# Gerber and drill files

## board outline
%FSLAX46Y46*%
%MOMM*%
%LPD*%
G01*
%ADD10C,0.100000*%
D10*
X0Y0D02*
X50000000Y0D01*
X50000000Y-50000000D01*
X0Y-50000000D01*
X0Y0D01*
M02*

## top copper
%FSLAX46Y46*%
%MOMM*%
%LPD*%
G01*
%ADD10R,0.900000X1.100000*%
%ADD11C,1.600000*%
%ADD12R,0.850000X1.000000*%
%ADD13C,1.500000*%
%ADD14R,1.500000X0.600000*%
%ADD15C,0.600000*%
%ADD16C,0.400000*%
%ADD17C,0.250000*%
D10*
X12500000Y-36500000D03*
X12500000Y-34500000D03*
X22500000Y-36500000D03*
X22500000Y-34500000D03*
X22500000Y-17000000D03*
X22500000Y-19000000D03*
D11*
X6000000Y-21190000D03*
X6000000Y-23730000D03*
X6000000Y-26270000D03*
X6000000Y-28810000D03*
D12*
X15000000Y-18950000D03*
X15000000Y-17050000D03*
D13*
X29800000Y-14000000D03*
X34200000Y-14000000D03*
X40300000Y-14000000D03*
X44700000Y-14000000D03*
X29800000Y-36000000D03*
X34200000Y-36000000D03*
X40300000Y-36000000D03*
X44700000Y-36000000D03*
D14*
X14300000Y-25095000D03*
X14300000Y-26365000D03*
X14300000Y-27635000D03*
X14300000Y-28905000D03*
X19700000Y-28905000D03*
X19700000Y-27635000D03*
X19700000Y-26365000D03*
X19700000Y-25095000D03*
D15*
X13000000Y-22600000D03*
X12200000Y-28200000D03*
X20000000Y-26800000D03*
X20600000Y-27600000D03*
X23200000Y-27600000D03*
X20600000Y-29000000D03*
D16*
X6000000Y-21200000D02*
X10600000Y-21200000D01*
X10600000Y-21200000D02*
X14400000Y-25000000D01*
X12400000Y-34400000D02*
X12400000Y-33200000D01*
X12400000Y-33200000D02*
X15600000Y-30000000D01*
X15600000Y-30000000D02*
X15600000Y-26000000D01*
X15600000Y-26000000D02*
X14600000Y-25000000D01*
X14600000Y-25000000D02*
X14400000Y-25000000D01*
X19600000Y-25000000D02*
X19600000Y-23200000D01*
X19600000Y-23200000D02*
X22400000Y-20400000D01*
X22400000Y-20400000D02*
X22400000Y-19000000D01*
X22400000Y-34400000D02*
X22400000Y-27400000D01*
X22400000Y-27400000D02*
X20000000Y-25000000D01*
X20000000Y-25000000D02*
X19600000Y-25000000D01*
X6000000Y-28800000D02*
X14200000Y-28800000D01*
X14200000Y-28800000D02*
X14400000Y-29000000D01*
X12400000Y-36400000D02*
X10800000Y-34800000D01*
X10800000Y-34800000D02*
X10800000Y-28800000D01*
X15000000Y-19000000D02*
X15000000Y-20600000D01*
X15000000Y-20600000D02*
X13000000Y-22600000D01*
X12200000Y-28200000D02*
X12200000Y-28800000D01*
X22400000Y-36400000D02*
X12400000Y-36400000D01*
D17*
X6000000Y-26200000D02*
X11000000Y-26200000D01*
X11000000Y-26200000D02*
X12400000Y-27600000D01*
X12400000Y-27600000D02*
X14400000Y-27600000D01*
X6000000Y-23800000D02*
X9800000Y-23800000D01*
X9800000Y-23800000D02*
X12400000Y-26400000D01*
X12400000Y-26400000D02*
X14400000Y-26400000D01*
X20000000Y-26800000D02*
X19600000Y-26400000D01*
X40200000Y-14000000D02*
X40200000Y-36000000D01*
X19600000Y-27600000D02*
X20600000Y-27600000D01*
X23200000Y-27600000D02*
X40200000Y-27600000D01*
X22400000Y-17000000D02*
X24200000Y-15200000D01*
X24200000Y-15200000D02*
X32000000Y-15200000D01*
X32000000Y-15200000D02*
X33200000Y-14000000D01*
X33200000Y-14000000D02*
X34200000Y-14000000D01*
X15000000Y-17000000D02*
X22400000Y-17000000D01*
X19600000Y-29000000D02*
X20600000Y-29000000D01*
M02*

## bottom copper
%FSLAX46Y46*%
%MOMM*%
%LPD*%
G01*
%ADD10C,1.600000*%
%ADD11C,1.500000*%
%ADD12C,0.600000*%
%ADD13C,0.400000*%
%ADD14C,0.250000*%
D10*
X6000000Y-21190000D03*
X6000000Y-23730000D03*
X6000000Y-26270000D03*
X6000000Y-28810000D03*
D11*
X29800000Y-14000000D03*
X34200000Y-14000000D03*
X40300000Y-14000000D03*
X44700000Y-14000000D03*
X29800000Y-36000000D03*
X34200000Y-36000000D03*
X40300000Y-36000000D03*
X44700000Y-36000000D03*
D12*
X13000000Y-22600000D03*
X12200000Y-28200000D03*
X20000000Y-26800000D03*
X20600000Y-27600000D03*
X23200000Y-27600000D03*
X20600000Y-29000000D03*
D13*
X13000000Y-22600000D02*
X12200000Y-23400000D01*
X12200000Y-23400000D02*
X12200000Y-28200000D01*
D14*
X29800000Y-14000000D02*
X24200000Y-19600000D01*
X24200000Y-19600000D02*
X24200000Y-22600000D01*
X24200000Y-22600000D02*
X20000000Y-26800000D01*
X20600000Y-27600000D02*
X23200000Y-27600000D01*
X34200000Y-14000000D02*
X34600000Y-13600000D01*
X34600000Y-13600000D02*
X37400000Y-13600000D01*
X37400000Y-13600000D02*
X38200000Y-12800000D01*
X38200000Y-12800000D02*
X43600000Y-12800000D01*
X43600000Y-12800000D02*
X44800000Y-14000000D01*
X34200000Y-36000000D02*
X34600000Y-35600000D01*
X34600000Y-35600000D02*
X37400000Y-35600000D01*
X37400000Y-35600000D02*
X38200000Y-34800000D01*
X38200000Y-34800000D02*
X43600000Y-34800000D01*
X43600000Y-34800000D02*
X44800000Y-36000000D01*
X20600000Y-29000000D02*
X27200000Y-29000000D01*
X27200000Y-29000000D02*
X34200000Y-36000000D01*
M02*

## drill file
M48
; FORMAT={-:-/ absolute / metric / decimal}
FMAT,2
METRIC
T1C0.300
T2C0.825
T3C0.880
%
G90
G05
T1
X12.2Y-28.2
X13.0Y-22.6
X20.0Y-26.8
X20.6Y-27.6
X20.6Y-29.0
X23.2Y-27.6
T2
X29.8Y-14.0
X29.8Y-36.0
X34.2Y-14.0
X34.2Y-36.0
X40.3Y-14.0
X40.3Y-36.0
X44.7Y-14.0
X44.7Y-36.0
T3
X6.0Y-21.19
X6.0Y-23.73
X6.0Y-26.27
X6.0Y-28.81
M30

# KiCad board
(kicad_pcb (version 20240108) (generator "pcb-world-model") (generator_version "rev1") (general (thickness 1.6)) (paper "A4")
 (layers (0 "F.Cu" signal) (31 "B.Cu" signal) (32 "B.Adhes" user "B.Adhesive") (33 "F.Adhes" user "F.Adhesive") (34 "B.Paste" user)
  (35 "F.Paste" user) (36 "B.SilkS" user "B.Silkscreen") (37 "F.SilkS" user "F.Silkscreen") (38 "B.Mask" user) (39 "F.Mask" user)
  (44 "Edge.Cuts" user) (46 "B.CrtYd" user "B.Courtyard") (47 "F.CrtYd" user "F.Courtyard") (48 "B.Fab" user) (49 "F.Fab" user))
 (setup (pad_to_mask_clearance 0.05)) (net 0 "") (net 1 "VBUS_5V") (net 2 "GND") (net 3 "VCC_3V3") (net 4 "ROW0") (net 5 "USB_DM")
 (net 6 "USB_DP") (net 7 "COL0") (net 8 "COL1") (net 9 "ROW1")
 (gr_rect (start 0.0 0.0) (end 50.0000 50.0000) (stroke (width 0.1) (type default)) (fill none) (layer "Edge.Cuts"))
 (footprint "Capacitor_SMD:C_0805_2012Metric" (layer "F.Cu") (at 12.5000 35.5000 90)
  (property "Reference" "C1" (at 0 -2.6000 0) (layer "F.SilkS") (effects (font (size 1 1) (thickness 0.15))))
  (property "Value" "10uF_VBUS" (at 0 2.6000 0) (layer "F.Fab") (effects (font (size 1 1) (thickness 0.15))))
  (pad "1" smd rect (at -1.0000 0.0000) (size 0.9000 1.1000) (layers "F.Cu" "F.Paste" "F.Mask") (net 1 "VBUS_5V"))
  (pad "2" smd rect (at 1.0000 0.0000) (size 0.9000 1.1000) (layers "F.Cu" "F.Paste" "F.Mask") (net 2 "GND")))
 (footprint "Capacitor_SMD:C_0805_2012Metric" (layer "F.Cu") (at 22.5000 35.5000 90)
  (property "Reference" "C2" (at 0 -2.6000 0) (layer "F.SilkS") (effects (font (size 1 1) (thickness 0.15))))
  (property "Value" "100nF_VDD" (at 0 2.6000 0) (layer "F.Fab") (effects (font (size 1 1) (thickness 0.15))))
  (pad "1" smd rect (at -1.0000 0.0000) (size 0.9000 1.1000) (layers "F.Cu" "F.Paste" "F.Mask") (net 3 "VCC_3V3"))
  (pad "2" smd rect (at 1.0000 0.0000) (size 0.9000 1.1000) (layers "F.Cu" "F.Paste" "F.Mask") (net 2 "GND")))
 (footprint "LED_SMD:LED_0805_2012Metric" (layer "F.Cu") (at 22.5000 18.0000 270)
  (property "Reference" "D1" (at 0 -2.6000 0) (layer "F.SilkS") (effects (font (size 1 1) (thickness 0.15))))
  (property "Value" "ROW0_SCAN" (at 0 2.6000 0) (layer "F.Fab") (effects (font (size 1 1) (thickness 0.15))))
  (pad "1" smd rect (at -1.0000 0.0000) (size 0.9000 1.1000) (layers "F.Cu" "F.Paste" "F.Mask") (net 3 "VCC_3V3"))
  (pad "2" smd rect (at 1.0000 0.0000) (size 0.9000 1.1000) (layers "F.Cu" "F.Paste" "F.Mask") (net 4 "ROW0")))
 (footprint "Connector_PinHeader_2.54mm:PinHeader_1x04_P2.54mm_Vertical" (layer "F.Cu") (at 6.0000 25.0000 0) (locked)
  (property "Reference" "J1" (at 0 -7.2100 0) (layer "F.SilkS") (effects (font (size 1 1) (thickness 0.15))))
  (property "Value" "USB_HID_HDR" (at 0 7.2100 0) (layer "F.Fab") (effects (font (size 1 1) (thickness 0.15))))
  (pad "1" thru_hole circle (at 0.0000 -3.8100) (size 1.6000 1.6000) (drill 0.8800) (layers "*.Cu" "*.Mask") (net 1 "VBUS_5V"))
  (pad "2" thru_hole circle (at 0.0000 -1.2700) (size 1.6000 1.6000) (drill 0.8800) (layers "*.Cu" "*.Mask") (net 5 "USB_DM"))
  (pad "3" thru_hole circle (at 0.0000 1.2700) (size 1.6000 1.6000) (drill 0.8800) (layers "*.Cu" "*.Mask") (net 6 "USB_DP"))
  (pad "4" thru_hole circle (at 0.0000 3.8100) (size 1.6000 1.6000) (drill 0.8800) (layers "*.Cu" "*.Mask") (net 2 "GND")))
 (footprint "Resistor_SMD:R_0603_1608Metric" (layer "F.Cu") (at 15.0000 18.0000 90)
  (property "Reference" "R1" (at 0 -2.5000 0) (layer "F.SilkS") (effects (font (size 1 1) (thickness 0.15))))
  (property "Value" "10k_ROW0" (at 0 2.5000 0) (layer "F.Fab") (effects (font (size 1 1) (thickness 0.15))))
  (pad "1" smd rect (at -0.9500 0.0000) (size 0.8500 1.0000) (layers "F.Cu" "F.Paste" "F.Mask") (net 4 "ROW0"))
  (pad "2" smd rect (at 0.9500 0.0000) (size 0.8500 1.0000) (layers "F.Cu" "F.Paste" "F.Mask") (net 2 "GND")))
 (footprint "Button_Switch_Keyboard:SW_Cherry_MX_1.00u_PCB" (layer "F.Cu") (at 32.0000 14.0000 0) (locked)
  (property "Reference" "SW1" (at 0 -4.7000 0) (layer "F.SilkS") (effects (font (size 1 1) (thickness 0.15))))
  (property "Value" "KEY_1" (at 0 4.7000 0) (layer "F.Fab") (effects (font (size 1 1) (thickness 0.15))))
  (pad "1" thru_hole circle (at -2.2000 0.0000) (size 1.5000 1.5000) (drill 0.8250) (layers "*.Cu" "*.Mask") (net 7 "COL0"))
  (pad "2" thru_hole circle (at 2.2000 0.0000) (size 1.5000 1.5000) (drill 0.8250) (layers "*.Cu" "*.Mask") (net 4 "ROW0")))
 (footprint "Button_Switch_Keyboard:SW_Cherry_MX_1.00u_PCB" (layer "F.Cu") (at 42.5000 14.0000 0) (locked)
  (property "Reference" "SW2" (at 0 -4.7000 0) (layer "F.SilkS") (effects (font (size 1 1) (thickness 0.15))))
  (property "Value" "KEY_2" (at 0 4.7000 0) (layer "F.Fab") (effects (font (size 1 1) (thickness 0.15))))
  (pad "1" thru_hole circle (at -2.2000 0.0000) (size 1.5000 1.5000) (drill 0.8250) (layers "*.Cu" "*.Mask") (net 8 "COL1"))
  (pad "2" thru_hole circle (at 2.2000 0.0000) (size 1.5000 1.5000) (drill 0.8250) (layers "*.Cu" "*.Mask") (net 4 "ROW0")))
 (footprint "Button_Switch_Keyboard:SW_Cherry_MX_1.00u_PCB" (layer "F.Cu") (at 32.0000 36.0000 0) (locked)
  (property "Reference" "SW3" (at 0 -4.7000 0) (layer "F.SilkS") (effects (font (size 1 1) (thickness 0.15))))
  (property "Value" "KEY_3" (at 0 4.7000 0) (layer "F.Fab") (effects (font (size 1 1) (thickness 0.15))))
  (pad "1" thru_hole circle (at -2.2000 0.0000) (size 1.5000 1.5000) (drill 0.8250) (layers "*.Cu" "*.Mask") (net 7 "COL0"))
  (pad "2" thru_hole circle (at 2.2000 0.0000) (size 1.5000 1.5000) (drill 0.8250) (layers "*.Cu" "*.Mask") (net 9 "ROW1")))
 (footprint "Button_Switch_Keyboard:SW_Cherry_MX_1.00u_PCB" (layer "F.Cu") (at 42.5000 36.0000 0) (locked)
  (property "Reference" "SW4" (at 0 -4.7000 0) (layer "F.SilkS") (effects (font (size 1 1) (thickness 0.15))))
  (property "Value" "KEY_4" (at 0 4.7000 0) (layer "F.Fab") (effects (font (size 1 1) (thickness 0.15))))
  (pad "1" thru_hole circle (at -2.2000 0.0000) (size 1.5000 1.5000) (drill 0.8250) (layers "*.Cu" "*.Mask") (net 8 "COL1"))
  (pad "2" thru_hole circle (at 2.2000 0.0000) (size 1.5000 1.5000) (drill 0.8250) (layers "*.Cu" "*.Mask") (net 9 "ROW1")))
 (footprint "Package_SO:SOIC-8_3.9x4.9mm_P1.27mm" (layer "F.Cu") (at 17.0000 27.0000 0)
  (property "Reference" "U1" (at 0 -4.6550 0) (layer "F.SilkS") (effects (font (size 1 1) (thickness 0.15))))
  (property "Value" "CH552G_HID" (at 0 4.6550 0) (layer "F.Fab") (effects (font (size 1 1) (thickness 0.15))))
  (pad "1" smd rect (at -2.7000 -1.9050) (size 1.5000 0.6000) (layers "F.Cu" "F.Paste" "F.Mask") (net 1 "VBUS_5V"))
  (pad "2" smd rect (at -2.7000 -0.6350) (size 1.5000 0.6000) (layers "F.Cu" "F.Paste" "F.Mask") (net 5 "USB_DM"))
  (pad "3" smd rect (at -2.7000 0.6350) (size 1.5000 0.6000) (layers "F.Cu" "F.Paste" "F.Mask") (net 6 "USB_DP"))
  (pad "4" smd rect (at -2.7000 1.9050) (size 1.5000 0.6000) (layers "F.Cu" "F.Paste" "F.Mask") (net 2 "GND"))
  (pad "5" smd rect (at 2.7000 1.9050) (size 1.5000 0.6000) (layers "F.Cu" "F.Paste" "F.Mask") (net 9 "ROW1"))
  (pad "6" smd rect (at 2.7000 0.6350) (size 1.5000 0.6000) (layers "F.Cu" "F.Paste" "F.Mask") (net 8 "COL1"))
  (pad "7" smd rect (at 2.7000 -0.6350) (size 1.5000 0.6000) (layers "F.Cu" "F.Paste" "F.Mask") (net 7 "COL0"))
  (pad "8" smd rect (at 2.7000 -1.9050) (size 1.5000 0.6000) (layers "F.Cu" "F.Paste" "F.Mask") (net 3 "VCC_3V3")))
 (segment (start 6.0000 21.2000) (end 10.6000 21.2000) (width 0.4000) (layer "F.Cu") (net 1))
 (segment (start 10.6000 21.2000) (end 14.4000 25.0000) (width 0.4000) (layer "F.Cu") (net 1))
 (segment (start 12.4000 34.4000) (end 12.4000 33.2000) (width 0.4000) (layer "F.Cu") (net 1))
 (segment (start 12.4000 33.2000) (end 15.6000 30.0000) (width 0.4000) (layer "F.Cu") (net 1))
 (segment (start 15.6000 30.0000) (end 15.6000 26.0000) (width 0.4000) (layer "F.Cu") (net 1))
 (segment (start 15.6000 26.0000) (end 14.6000 25.0000) (width 0.4000) (layer "F.Cu") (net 1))
 (segment (start 14.6000 25.0000) (end 14.4000 25.0000) (width 0.4000) (layer "F.Cu") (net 1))
 (segment (start 19.6000 25.0000) (end 19.6000 23.2000) (width 0.4000) (layer "F.Cu") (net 3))
 (segment (start 19.6000 23.2000) (end 22.4000 20.4000) (width 0.4000) (layer "F.Cu") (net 3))
 (segment (start 22.4000 20.4000) (end 22.4000 19.0000) (width 0.4000) (layer "F.Cu") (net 3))
 (segment (start 22.4000 34.4000) (end 22.4000 27.4000) (width 0.4000) (layer "F.Cu") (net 3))
 (segment (start 22.4000 27.4000) (end 20.0000 25.0000) (width 0.4000) (layer "F.Cu") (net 3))
 (segment (start 20.0000 25.0000) (end 19.6000 25.0000) (width 0.4000) (layer "F.Cu") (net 3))
 (segment (start 6.0000 28.8000) (end 14.2000 28.8000) (width 0.4000) (layer "F.Cu") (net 2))
 (segment (start 14.2000 28.8000) (end 14.4000 29.0000) (width 0.4000) (layer "F.Cu") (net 2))
 (segment (start 12.4000 36.4000) (end 10.8000 34.8000) (width 0.4000) (layer "F.Cu") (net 2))
 (segment (start 10.8000 34.8000) (end 10.8000 28.8000) (width 0.4000) (layer "F.Cu") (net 2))
 (segment (start 15.0000 19.0000) (end 15.0000 20.6000) (width 0.4000) (layer "F.Cu") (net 2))
 (segment (start 15.0000 20.6000) (end 13.0000 22.6000) (width 0.4000) (layer "F.Cu") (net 2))
 (segment (start 13.0000 22.6000) (end 12.2000 23.4000) (width 0.4000) (layer "B.Cu") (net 2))
 (segment (start 12.2000 23.4000) (end 12.2000 28.2000) (width 0.4000) (layer "B.Cu") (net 2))
 (segment (start 12.2000 28.2000) (end 12.2000 28.8000) (width 0.4000) (layer "F.Cu") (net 2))
 (segment (start 22.4000 36.4000) (end 12.4000 36.4000) (width 0.4000) (layer "F.Cu") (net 2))
 (segment (start 6.0000 26.2000) (end 11.0000 26.2000) (width 0.2500) (layer "F.Cu") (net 6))
 (segment (start 11.0000 26.2000) (end 12.4000 27.6000) (width 0.2500) (layer "F.Cu") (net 6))
 (segment (start 12.4000 27.6000) (end 14.4000 27.6000) (width 0.2500) (layer "F.Cu") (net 6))
 (segment (start 6.0000 23.8000) (end 9.8000 23.8000) (width 0.2500) (layer "F.Cu") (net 5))
 (segment (start 9.8000 23.8000) (end 12.4000 26.4000) (width 0.2500) (layer "F.Cu") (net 5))
 (segment (start 12.4000 26.4000) (end 14.4000 26.4000) (width 0.2500) (layer "F.Cu") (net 5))
 (segment (start 29.8000 14.0000) (end 24.2000 19.6000) (width 0.2500) (layer "B.Cu") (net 7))
 (segment (start 24.2000 19.6000) (end 24.2000 22.6000) (width 0.2500) (layer "B.Cu") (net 7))
 (segment (start 24.2000 22.6000) (end 20.0000 26.8000) (width 0.2500) (layer "B.Cu") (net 7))
 (segment (start 20.0000 26.8000) (end 19.6000 26.4000) (width 0.2500) (layer "F.Cu") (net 7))
 (segment (start 40.2000 14.0000) (end 40.2000 36.0000) (width 0.2500) (layer "F.Cu") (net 8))
 (segment (start 19.6000 27.6000) (end 20.6000 27.6000) (width 0.2500) (layer "F.Cu") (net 8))
 (segment (start 20.6000 27.6000) (end 23.2000 27.6000) (width 0.2500) (layer "B.Cu") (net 8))
 (segment (start 23.2000 27.6000) (end 40.2000 27.6000) (width 0.2500) (layer "F.Cu") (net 8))
 (segment (start 34.2000 14.0000) (end 34.6000 13.6000) (width 0.2500) (layer "B.Cu") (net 4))
 (segment (start 34.6000 13.6000) (end 37.4000 13.6000) (width 0.2500) (layer "B.Cu") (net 4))
 (segment (start 37.4000 13.6000) (end 38.2000 12.8000) (width 0.2500) (layer "B.Cu") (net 4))
 (segment (start 38.2000 12.8000) (end 43.6000 12.8000) (width 0.2500) (layer "B.Cu") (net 4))
 (segment (start 43.6000 12.8000) (end 44.8000 14.0000) (width 0.2500) (layer "B.Cu") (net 4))
 (segment (start 22.4000 17.0000) (end 24.2000 15.2000) (width 0.2500) (layer "F.Cu") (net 4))
 (segment (start 24.2000 15.2000) (end 32.0000 15.2000) (width 0.2500) (layer "F.Cu") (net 4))
 (segment (start 32.0000 15.2000) (end 33.2000 14.0000) (width 0.2500) (layer "F.Cu") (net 4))
 (segment (start 33.2000 14.0000) (end 34.2000 14.0000) (width 0.2500) (layer "F.Cu") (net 4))
 (segment (start 15.0000 17.0000) (end 22.4000 17.0000) (width 0.2500) (layer "F.Cu") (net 4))
 (segment (start 34.2000 36.0000) (end 34.6000 35.6000) (width 0.2500) (layer "B.Cu") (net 9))
 (segment (start 34.6000 35.6000) (end 37.4000 35.6000) (width 0.2500) (layer "B.Cu") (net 9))
 (segment (start 37.4000 35.6000) (end 38.2000 34.8000) (width 0.2500) (layer "B.Cu") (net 9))
 (segment (start 38.2000 34.8000) (end 43.6000 34.8000) (width 0.2500) (layer "B.Cu") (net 9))
 (segment (start 43.6000 34.8000) (end 44.8000 36.0000) (width 0.2500) (layer "B.Cu") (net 9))
 (segment (start 19.6000 29.0000) (end 20.6000 29.0000) (width 0.2500) (layer "F.Cu") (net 9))
 (segment (start 20.6000 29.0000) (end 27.2000 29.0000) (width 0.2500) (layer "B.Cu") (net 9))
 (segment (start 27.2000 29.0000) (end 34.2000 36.0000) (width 0.2500) (layer "B.Cu") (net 9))
 (via (at 13.0000 22.6000) (size 0.6000) (drill 0.3000) (layers "F.Cu" "B.Cu") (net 2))
 (via (at 12.2000 28.2000) (size 0.6000) (drill 0.3000) (layers "F.Cu" "B.Cu") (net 2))
 (via (at 20.0000 26.8000) (size 0.6000) (drill 0.3000) (layers "F.Cu" "B.Cu") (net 7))
 (via (at 20.6000 27.6000) (size 0.6000) (drill 0.3000) (layers "F.Cu" "B.Cu") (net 8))
 (via (at 23.2000 27.6000) (size 0.6000) (drill 0.3000) (layers "F.Cu" "B.Cu") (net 8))
 (via (at 20.6000 29.0000) (size 0.6000) (drill 0.3000) (layers "F.Cu" "B.Cu") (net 9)))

